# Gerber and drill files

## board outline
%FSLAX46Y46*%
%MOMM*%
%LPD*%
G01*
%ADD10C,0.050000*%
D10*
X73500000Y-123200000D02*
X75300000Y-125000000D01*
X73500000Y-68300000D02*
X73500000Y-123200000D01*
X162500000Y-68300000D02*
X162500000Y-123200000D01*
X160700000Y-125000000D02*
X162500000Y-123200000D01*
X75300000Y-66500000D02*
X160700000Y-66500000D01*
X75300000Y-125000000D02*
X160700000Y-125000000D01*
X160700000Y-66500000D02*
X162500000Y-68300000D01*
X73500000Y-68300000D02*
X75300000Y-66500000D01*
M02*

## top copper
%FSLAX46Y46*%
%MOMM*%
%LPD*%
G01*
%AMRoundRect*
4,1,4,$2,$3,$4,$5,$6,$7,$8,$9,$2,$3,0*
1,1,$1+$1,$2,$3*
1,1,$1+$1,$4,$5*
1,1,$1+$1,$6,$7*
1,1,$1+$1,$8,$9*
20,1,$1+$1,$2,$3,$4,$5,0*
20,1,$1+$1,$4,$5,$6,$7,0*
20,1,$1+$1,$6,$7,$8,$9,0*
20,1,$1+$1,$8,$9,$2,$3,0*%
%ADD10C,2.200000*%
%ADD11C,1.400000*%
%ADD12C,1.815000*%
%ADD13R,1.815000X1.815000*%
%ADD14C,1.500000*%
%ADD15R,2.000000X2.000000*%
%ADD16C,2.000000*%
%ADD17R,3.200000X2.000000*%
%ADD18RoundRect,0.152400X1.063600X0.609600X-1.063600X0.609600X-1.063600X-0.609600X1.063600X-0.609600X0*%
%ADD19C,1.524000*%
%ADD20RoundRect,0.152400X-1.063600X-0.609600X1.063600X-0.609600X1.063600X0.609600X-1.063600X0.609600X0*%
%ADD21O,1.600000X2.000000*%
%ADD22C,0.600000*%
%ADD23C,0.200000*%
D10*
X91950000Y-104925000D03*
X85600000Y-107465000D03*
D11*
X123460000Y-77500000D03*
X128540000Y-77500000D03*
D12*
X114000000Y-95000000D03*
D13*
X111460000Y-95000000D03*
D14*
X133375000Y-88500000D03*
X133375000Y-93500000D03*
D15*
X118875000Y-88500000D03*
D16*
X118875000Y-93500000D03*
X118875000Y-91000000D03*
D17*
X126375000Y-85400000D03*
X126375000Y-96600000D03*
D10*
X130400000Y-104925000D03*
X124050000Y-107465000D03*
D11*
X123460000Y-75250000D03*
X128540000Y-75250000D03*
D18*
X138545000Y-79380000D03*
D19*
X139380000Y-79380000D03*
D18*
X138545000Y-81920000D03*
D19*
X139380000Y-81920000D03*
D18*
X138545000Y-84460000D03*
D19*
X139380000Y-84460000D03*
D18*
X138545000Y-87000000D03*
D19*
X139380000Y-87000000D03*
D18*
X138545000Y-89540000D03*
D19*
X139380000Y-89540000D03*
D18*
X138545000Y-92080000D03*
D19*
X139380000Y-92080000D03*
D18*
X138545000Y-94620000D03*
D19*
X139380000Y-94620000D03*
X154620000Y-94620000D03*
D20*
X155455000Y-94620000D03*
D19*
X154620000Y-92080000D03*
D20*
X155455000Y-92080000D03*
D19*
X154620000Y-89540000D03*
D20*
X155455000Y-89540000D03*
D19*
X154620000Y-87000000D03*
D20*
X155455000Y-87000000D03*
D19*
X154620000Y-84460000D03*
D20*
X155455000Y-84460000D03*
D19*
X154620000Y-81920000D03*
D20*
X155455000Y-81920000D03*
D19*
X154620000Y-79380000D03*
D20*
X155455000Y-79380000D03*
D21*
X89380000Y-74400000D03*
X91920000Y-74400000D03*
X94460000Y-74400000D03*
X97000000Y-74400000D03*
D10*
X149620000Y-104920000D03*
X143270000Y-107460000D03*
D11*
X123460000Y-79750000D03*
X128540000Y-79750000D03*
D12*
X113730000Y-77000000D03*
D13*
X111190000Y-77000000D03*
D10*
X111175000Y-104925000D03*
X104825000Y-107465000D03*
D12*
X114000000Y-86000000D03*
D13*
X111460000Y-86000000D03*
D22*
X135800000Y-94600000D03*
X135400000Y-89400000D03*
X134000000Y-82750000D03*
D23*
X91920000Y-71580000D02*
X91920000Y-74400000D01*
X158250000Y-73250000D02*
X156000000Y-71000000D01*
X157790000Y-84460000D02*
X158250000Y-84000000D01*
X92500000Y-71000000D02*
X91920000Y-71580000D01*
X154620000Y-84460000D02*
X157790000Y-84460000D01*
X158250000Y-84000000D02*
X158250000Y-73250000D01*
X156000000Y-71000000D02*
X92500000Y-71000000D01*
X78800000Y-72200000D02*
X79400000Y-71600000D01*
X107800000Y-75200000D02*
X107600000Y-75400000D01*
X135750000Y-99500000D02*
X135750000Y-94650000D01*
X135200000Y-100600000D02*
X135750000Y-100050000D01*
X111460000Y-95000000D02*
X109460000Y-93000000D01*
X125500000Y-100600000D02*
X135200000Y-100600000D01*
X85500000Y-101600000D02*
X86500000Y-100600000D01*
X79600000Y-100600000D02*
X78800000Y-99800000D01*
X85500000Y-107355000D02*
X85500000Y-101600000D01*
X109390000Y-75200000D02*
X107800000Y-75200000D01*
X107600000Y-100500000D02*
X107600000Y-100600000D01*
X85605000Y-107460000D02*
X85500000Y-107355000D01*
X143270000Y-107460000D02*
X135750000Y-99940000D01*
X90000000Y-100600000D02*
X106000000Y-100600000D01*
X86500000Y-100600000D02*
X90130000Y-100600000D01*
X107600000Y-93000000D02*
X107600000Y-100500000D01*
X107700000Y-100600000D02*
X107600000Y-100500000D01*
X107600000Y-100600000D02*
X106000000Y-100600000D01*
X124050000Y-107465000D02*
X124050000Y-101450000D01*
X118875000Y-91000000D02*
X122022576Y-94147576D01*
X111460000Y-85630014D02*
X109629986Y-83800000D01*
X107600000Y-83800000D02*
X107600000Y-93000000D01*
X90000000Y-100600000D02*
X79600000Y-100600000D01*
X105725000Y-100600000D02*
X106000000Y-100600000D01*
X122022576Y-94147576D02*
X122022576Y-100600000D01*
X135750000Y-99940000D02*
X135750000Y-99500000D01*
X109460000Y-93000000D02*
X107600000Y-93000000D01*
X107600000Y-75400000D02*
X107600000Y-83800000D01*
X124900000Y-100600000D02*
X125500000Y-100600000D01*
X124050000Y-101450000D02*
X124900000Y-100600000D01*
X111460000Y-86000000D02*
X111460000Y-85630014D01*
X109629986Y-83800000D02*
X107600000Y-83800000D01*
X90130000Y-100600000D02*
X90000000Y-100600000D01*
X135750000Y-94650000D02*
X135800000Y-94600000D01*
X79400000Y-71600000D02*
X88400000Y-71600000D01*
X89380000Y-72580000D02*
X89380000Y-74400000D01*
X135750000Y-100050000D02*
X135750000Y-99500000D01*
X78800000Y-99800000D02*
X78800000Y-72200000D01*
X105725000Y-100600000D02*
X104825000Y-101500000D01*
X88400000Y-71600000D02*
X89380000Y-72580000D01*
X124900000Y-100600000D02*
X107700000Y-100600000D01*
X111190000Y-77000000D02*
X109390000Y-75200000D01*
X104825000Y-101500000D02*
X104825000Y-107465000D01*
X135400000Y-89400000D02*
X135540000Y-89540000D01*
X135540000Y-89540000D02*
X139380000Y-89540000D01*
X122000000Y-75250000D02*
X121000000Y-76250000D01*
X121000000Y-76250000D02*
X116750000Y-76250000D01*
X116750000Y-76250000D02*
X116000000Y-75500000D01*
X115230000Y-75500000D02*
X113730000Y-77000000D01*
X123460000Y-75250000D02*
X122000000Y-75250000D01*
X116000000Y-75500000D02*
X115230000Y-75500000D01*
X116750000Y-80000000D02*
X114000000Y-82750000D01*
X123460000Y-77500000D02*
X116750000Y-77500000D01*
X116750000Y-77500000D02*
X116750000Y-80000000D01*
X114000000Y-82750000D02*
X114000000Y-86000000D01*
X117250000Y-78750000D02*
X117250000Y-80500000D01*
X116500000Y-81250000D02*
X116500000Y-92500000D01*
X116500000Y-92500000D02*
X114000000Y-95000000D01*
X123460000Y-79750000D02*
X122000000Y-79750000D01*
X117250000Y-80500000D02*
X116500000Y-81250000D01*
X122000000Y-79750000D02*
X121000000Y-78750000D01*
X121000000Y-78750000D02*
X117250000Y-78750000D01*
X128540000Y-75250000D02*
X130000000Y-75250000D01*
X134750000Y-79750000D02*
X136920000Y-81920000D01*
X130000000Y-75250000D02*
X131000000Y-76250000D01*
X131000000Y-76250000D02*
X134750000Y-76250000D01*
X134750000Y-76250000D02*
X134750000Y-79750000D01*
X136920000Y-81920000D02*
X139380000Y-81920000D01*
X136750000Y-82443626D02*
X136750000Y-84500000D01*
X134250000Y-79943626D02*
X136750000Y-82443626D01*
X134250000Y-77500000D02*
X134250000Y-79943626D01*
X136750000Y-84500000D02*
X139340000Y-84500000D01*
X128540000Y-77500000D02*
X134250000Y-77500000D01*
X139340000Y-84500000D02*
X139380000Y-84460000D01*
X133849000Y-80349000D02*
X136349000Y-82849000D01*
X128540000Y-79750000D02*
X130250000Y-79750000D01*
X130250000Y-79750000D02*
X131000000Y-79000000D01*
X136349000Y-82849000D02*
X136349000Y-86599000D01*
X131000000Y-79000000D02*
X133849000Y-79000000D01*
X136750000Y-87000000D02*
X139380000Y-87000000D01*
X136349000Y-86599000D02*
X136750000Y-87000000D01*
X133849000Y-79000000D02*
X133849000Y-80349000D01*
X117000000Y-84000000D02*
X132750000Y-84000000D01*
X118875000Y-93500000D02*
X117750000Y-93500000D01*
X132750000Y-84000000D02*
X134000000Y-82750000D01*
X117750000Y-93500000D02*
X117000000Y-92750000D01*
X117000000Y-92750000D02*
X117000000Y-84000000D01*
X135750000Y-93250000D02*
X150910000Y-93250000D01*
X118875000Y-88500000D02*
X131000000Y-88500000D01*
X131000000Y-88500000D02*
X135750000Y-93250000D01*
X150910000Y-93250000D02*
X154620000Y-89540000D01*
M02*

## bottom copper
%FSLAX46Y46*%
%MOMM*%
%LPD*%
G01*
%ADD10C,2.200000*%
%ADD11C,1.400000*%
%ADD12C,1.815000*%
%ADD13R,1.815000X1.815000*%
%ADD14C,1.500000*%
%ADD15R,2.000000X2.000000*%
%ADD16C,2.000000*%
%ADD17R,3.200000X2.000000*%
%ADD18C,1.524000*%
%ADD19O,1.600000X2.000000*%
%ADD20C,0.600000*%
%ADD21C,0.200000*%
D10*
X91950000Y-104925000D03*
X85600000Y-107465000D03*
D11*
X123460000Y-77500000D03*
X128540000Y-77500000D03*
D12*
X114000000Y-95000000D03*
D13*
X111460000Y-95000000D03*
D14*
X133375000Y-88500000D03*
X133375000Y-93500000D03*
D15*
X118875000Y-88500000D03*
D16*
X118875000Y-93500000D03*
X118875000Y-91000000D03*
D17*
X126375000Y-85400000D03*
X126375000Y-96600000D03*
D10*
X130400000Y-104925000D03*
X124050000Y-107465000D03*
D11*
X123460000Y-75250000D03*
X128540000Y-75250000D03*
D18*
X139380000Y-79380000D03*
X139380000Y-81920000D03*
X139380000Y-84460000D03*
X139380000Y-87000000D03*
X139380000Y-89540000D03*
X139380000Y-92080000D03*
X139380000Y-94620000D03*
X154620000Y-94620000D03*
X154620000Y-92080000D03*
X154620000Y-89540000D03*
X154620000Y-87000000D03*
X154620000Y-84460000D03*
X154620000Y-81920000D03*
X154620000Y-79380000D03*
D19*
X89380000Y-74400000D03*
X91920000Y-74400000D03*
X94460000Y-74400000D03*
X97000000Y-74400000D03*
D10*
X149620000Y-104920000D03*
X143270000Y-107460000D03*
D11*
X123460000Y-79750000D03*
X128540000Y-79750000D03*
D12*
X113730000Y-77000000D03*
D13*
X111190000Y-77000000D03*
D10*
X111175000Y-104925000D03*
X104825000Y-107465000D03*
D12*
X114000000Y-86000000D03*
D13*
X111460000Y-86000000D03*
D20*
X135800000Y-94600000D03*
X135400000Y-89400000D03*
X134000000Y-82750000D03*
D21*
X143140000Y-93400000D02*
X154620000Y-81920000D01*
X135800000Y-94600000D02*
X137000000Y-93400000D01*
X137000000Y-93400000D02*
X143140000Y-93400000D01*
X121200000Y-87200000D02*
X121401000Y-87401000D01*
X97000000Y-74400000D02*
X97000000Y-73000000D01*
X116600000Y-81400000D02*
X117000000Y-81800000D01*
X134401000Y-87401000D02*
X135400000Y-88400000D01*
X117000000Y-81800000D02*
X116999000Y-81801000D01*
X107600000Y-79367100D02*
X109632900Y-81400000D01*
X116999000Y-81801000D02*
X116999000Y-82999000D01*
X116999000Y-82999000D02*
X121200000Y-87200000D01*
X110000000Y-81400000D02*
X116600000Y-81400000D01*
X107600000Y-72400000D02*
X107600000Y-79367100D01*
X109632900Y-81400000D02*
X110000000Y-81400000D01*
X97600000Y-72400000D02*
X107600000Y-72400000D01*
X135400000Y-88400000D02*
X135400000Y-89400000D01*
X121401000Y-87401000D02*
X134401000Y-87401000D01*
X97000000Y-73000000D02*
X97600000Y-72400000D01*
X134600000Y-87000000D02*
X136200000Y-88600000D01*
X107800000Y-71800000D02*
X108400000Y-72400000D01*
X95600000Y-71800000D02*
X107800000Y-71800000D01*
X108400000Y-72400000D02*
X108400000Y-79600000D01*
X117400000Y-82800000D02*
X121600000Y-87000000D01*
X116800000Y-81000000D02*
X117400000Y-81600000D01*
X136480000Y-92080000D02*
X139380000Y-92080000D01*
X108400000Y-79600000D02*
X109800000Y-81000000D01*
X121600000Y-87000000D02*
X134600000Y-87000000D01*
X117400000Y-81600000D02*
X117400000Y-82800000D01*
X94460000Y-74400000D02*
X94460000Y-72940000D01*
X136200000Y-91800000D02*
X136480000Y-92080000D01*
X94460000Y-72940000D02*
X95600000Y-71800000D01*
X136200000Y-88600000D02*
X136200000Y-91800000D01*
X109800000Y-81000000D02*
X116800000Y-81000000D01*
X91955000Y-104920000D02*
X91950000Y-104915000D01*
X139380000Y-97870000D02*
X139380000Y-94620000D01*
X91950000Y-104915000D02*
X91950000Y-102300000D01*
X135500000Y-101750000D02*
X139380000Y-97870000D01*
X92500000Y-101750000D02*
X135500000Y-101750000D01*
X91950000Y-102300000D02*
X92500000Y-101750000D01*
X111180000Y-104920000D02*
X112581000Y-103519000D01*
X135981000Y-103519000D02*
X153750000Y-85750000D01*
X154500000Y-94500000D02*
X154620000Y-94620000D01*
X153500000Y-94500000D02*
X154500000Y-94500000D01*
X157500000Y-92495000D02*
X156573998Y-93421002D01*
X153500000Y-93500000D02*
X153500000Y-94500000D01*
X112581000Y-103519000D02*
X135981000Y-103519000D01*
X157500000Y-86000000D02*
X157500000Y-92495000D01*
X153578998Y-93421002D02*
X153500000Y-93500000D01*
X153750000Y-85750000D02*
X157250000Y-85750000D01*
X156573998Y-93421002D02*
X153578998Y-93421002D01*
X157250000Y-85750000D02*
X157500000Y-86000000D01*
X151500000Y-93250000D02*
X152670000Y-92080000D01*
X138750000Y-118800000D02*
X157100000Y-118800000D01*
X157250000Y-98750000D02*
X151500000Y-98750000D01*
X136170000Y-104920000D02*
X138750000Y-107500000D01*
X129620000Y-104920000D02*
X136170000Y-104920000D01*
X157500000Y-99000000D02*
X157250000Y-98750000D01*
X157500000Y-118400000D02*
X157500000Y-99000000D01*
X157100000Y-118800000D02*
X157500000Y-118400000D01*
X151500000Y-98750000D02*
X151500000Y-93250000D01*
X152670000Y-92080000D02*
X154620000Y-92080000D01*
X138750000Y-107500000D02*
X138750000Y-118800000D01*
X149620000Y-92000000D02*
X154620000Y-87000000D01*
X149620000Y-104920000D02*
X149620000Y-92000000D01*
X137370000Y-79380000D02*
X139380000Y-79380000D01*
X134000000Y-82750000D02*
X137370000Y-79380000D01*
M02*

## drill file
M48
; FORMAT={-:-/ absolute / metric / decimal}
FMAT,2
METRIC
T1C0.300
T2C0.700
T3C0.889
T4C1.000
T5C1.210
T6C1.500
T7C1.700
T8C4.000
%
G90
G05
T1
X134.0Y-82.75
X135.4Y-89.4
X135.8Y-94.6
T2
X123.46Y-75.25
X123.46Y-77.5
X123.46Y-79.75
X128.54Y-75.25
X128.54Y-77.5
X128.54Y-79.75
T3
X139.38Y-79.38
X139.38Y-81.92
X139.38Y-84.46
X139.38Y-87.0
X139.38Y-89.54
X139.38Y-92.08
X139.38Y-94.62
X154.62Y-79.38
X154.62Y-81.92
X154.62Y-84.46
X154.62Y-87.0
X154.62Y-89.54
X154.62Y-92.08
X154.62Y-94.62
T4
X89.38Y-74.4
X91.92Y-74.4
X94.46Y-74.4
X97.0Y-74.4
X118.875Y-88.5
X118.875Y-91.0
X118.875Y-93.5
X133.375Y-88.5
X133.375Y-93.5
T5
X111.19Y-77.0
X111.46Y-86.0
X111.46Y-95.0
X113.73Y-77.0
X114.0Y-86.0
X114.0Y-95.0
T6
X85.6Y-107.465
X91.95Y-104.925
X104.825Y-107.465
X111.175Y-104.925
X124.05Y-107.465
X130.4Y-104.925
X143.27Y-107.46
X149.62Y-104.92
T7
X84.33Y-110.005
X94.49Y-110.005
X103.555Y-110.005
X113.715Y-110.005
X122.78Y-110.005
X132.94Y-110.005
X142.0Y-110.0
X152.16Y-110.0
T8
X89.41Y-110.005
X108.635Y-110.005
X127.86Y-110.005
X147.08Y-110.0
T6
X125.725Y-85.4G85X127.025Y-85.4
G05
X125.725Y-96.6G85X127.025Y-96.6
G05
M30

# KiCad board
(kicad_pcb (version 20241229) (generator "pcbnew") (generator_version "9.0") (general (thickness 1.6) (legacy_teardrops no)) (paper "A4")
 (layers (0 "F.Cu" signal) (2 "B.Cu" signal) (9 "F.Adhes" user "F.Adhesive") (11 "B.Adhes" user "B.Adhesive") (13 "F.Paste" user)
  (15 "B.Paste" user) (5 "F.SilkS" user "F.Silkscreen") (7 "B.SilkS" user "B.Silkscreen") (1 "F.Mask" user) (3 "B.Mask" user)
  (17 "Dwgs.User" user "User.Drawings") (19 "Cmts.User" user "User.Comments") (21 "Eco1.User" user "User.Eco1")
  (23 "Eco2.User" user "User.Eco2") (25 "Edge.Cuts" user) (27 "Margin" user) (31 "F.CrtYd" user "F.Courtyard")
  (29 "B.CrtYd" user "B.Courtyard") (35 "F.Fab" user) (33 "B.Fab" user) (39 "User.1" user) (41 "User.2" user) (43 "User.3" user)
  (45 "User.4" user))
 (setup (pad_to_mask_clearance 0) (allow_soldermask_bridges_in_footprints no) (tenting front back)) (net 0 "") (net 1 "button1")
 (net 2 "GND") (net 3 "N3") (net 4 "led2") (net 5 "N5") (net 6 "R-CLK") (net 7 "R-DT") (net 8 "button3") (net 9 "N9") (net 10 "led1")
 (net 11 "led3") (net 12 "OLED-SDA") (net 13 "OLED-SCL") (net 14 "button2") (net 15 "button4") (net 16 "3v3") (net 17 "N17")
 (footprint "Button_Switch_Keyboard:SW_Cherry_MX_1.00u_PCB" (layer "F.Cu") (at 91.95 104.925)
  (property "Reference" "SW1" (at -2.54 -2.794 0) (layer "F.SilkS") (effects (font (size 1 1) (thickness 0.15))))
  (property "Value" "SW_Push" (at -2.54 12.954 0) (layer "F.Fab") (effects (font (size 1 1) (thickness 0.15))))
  (pad "" np_thru_hole circle (at -7.62 5.08) (size 1.7 1.7) (drill 1.7) (layers "*.Cu" "*.Mask"))
  (pad "" np_thru_hole circle (at -2.54 5.08) (size 4 4) (drill 4) (layers "*.Cu" "*.Mask"))
  (pad "" np_thru_hole circle (at 2.54 5.08) (size 1.7 1.7) (drill 1.7) (layers "*.Cu" "*.Mask"))
  (pad "1" thru_hole circle (at 0 0) (size 2.2 2.2) (drill 1.5) (layers "*.Cu" "*.Mask") (remove_unused_layers no) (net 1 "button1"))
  (pad "2" thru_hole circle (at -6.35 2.54) (size 2.2 2.2) (drill 1.5) (layers "*.Cu" "*.Mask") (remove_unused_layers no) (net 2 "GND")))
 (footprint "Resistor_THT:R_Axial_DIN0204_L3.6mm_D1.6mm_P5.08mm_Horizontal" (layer "F.Cu") (at 123.46 77.5)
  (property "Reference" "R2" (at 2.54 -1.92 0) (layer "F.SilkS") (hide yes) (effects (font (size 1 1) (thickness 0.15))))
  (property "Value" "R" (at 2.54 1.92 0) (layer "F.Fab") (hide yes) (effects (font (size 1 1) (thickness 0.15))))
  (pad "1" thru_hole circle (at 0 0) (size 1.4 1.4) (drill 0.7) (layers "*.Cu" "*.Mask") (remove_unused_layers no) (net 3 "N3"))
  (pad "2" thru_hole circle (at 5.08 0) (size 1.4 1.4) (drill 0.7) (layers "*.Cu" "*.Mask") (remove_unused_layers no) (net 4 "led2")))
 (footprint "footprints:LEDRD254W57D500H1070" (layer "F.Cu") (at 112.73 95)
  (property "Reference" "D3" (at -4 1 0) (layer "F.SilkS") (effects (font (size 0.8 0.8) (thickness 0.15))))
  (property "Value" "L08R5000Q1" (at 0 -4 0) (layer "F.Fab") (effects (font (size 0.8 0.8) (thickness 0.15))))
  (pad "A" thru_hole circle (at 1.27 0) (size 1.815 1.815) (drill 1.21) (layers "*.Cu" "*.Mask") (remove_unused_layers no) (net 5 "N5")
   (solder_mask_margin 0.102))
  (pad "C" thru_hole rect (at -1.27 0) (size 1.815 1.815) (drill 1.21) (layers "*.Cu" "*.Mask") (remove_unused_layers no) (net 2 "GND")
   (solder_mask_margin 0.102)))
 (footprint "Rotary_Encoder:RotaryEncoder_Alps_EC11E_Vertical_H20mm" (layer "F.Cu") (at 118.875 88.5)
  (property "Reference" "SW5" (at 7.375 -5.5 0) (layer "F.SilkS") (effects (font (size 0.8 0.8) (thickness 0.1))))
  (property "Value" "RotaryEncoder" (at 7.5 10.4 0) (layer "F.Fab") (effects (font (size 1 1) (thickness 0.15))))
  (pad "" thru_hole circle (at 14.5 0) (size 1.5 1.5) (drill 1) (layers "*.Cu" "*.Mask") (remove_unused_layers no))
  (pad "" thru_hole circle (at 14.5 5) (size 1.5 1.5) (drill 1) (layers "*.Cu" "*.Mask") (remove_unused_layers no))
  (pad "A" thru_hole rect (at 0 0) (size 2 2) (drill 1) (layers "*.Cu" "*.Mask") (remove_unused_layers no) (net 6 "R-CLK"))
  (pad "B" thru_hole circle (at 0 5) (size 2 2) (drill 1) (layers "*.Cu" "*.Mask") (remove_unused_layers no) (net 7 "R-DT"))
  (pad "C" thru_hole circle (at 0 2.5) (size 2 2) (drill 1) (layers "*.Cu" "*.Mask") (remove_unused_layers no) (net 2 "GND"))
  (pad "MP" thru_hole rect (at 7.5 -3.1) (size 3.2 2) (drill oval 2.8 1.5) (layers "*.Cu" "*.Mask") (remove_unused_layers no))
  (pad "MP" thru_hole rect (at 7.5 8.1) (size 3.2 2) (drill oval 2.8 1.5) (layers "*.Cu" "*.Mask") (remove_unused_layers no)))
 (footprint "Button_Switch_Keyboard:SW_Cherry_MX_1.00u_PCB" (layer "F.Cu") (at 130.4 104.925)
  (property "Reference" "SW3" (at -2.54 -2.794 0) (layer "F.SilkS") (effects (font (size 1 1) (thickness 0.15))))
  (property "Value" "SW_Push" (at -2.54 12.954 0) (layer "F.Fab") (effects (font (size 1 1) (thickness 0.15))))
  (pad "" np_thru_hole circle (at -7.62 5.08) (size 1.7 1.7) (drill 1.7) (layers "*.Cu" "*.Mask"))
  (pad "" np_thru_hole circle (at -2.54 5.08) (size 4 4) (drill 4) (layers "*.Cu" "*.Mask"))
  (pad "" np_thru_hole circle (at 2.54 5.08) (size 1.7 1.7) (drill 1.7) (layers "*.Cu" "*.Mask"))
  (pad "1" thru_hole circle (at 0 0) (size 2.2 2.2) (drill 1.5) (layers "*.Cu" "*.Mask") (remove_unused_layers no) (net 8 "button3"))
  (pad "2" thru_hole circle (at -6.35 2.54) (size 2.2 2.2) (drill 1.5) (layers "*.Cu" "*.Mask") (remove_unused_layers no) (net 2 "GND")))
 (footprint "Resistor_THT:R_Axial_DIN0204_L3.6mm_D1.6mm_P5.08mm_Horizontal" (layer "F.Cu") (at 123.46 75.25)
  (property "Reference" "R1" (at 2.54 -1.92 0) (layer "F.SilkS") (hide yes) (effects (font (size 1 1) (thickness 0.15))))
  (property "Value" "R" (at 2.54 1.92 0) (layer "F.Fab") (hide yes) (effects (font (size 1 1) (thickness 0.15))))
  (pad "1" thru_hole circle (at 0 0) (size 1.4 1.4) (drill 0.7) (layers "*.Cu" "*.Mask") (remove_unused_layers no) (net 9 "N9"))
  (pad "2" thru_hole circle (at 5.08 0) (size 1.4 1.4) (drill 0.7) (layers "*.Cu" "*.Mask") (remove_unused_layers no) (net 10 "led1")))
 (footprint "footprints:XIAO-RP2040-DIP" (layer "F.Cu") (at 147 87)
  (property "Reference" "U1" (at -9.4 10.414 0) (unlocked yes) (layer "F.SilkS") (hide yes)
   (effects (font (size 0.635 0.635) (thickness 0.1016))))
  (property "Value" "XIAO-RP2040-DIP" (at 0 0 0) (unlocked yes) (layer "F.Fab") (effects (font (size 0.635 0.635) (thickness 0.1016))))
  (pad "1" smd roundrect (at -8.455 -7.62 180) (size 2.432 1.524) (layers "F.Cu" "F.Mask") (roundrect_rratio 0.1) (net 7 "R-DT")
   (thermal_bridge_angle 45))
  (pad "1" thru_hole circle (at -7.62 -7.62 180) (size 1.524 1.524) (drill 0.889) (layers "*.Cu" "*.Mask") (remove_unused_layers no)
   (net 7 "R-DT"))
  (pad "2" smd roundrect (at -8.455 -5.08 180) (size 2.432 1.524) (layers "F.Cu" "F.Mask") (roundrect_rratio 0.1) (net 10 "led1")
   (thermal_bridge_angle 45))
  (pad "2" thru_hole circle (at -7.62 -5.08 180) (size 1.524 1.524) (drill 0.889) (layers "*.Cu" "*.Mask") (remove_unused_layers no)
   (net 10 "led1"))
  (pad "3" smd roundrect (at -8.455 -2.54 180) (size 2.432 1.524) (layers "F.Cu" "F.Mask") (roundrect_rratio 0.1) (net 4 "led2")
   (thermal_bridge_angle 45))
  (pad "3" thru_hole circle (at -7.62 -2.54 180) (size 1.524 1.524) (drill 0.889) (layers "*.Cu" "*.Mask") (remove_unused_layers no)
   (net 4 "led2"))
  (pad "4" smd roundrect (at -8.455 0 180) (size 2.432 1.524) (layers "F.Cu" "F.Mask") (roundrect_rratio 0.1) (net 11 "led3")
   (thermal_bridge_angle 45))
  (pad "4" thru_hole circle (at -7.62 0 180) (size 1.524 1.524) (drill 0.889) (layers "*.Cu" "*.Mask") (remove_unused_layers no)
   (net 11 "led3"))
  (pad "5" smd roundrect (at -8.455 2.54 180) (size 2.432 1.524) (layers "F.Cu" "F.Mask") (roundrect_rratio 0.1) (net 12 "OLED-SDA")
   (thermal_bridge_angle 45))
  (pad "5" thru_hole circle (at -7.62 2.54 180) (size 1.524 1.524) (drill 0.889) (layers "*.Cu" "*.Mask") (remove_unused_layers no)
   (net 12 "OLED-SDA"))
  (pad "6" smd roundrect (at -8.455 5.08 180) (size 2.432 1.524) (layers "F.Cu" "F.Mask") (roundrect_rratio 0.1) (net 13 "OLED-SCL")
   (thermal_bridge_angle 45))
  (pad "6" thru_hole circle (at -7.62 5.08 180) (size 1.524 1.524) (drill 0.889) (layers "*.Cu" "*.Mask") (remove_unused_layers no)
   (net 13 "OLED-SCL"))
  (pad "7" smd roundrect (at -8.455 7.62 180) (size 2.432 1.524) (layers "F.Cu" "F.Mask") (roundrect_rratio 0.1) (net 1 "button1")
   (thermal_bridge_angle 45))
  (pad "7" thru_hole circle (at -7.62 7.62 180) (size 1.524 1.524) (drill 0.889) (layers "*.Cu" "*.Mask") (remove_unused_layers no)
   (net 1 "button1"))
  (pad "8" thru_hole circle (at 7.62 7.62) (size 1.524 1.524) (drill 0.889) (layers "*.Cu" "*.Mask") (remove_unused_layers no)
   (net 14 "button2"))
  (pad "8" smd roundrect (at 8.455 7.62) (size 2.432 1.524) (layers "F.Cu" "F.Mask") (roundrect_rratio 0.1) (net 14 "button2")
   (thermal_bridge_angle 45))
  (pad "9" thru_hole circle (at 7.62 5.08) (size 1.524 1.524) (drill 0.889) (layers "*.Cu" "*.Mask") (remove_unused_layers no)
   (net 8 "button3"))
  (pad "9" smd roundrect (at 8.455 5.08) (size 2.432 1.524) (layers "F.Cu" "F.Mask") (roundrect_rratio 0.1) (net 8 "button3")
   (thermal_bridge_angle 45))
  (pad "10" thru_hole circle (at 7.62 2.54) (size 1.524 1.524) (drill 0.889) (layers "*.Cu" "*.Mask") (remove_unused_layers no)
   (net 6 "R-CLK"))
  (pad "10" smd roundrect (at 8.455 2.54) (size 2.432 1.524) (layers "F.Cu" "F.Mask") (roundrect_rratio 0.1) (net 6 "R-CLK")
   (thermal_bridge_angle 45))
  (pad "11" thru_hole circle (at 7.62 0) (size 1.524 1.524) (drill 0.889) (layers "*.Cu" "*.Mask") (remove_unused_layers no)
   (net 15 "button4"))
  (pad "11" smd roundrect (at 8.455 0) (size 2.432 1.524) (layers "F.Cu" "F.Mask") (roundrect_rratio 0.1) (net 15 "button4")
   (thermal_bridge_angle 45))
  (pad "12" thru_hole circle (at 7.62 -2.54) (size 1.524 1.524) (drill 0.889) (layers "*.Cu" "*.Mask") (remove_unused_layers no)
   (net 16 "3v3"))
  (pad "12" smd roundrect (at 8.455 -2.54) (size 2.432 1.524) (layers "F.Cu" "F.Mask") (roundrect_rratio 0.1) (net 16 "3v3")
   (thermal_bridge_angle 45))
  (pad "13" thru_hole circle (at 7.62 -5.08) (size 1.524 1.524) (drill 0.889) (layers "*.Cu" "*.Mask") (remove_unused_layers no)
   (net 2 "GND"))
  (pad "13" smd roundrect (at 8.455 -5.08) (size 2.432 1.524) (layers "F.Cu" "F.Mask") (roundrect_rratio 0.1) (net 2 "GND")
   (thermal_bridge_angle 45))
  (pad "14" thru_hole circle (at 7.62 -7.62) (size 1.524 1.524) (drill 0.889) (layers "*.Cu" "*.Mask") (remove_unused_layers no)
   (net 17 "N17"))
  (pad "14" smd roundrect (at 8.455 -7.62) (size 2.432 1.524) (layers "F.Cu" "F.Mask") (roundrect_rratio 0.1) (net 17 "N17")
   (thermal_bridge_angle 45)))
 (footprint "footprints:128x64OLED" (layer "F.Cu") (at 93 85)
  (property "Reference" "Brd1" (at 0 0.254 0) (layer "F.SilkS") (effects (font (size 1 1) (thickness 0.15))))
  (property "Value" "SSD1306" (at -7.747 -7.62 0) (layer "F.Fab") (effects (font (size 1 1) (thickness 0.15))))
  (pad "1" thru_hole oval (at -3.62 -10.6 90) (size 2 1.6) (drill 1) (layers "*.Cu" "*.Mask") (remove_unused_layers no) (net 2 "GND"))
  (pad "2" thru_hole oval (at -1.08 -10.6 90) (size 2 1.6) (drill 1) (layers "*.Cu" "*.Mask") (remove_unused_layers no) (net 16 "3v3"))
  (pad "3" thru_hole oval (at 1.46 -10.6 90) (size 2 1.6) (drill 1) (layers "*.Cu" "*.Mask") (remove_unused_layers no) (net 13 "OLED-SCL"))
  (pad "4" thru_hole oval (at 4 -10.6 90) (size 2 1.6) (drill 1) (layers "*.Cu" "*.Mask") (remove_unused_layers no) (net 12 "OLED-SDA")))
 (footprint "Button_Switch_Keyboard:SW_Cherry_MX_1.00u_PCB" (layer "F.Cu") (at 149.62 104.92)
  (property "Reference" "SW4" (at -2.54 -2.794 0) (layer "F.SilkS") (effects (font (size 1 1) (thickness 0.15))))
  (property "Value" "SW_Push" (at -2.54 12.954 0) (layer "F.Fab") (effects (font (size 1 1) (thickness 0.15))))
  (pad "" np_thru_hole circle (at -7.62 5.08) (size 1.7 1.7) (drill 1.7) (layers "*.Cu" "*.Mask"))
  (pad "" np_thru_hole circle (at -2.54 5.08) (size 4 4) (drill 4) (layers "*.Cu" "*.Mask"))
  (pad "" np_thru_hole circle (at 2.54 5.08) (size 1.7 1.7) (drill 1.7) (layers "*.Cu" "*.Mask"))
  (pad "1" thru_hole circle (at 0 0) (size 2.2 2.2) (drill 1.5) (layers "*.Cu" "*.Mask") (remove_unused_layers no) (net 15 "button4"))
  (pad "2" thru_hole circle (at -6.35 2.54) (size 2.2 2.2) (drill 1.5) (layers "*.Cu" "*.Mask") (remove_unused_layers no) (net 2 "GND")))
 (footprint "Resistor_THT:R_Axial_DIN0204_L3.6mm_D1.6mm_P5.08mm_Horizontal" (layer "F.Cu") (at 123.46 79.75)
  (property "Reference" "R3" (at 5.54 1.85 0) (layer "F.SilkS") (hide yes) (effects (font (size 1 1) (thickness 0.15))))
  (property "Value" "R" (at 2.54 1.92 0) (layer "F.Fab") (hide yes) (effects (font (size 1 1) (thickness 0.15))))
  (pad "1" thru_hole circle (at 0 0) (size 1.4 1.4) (drill 0.7) (layers "*.Cu" "*.Mask") (remove_unused_layers no) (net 5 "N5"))
  (pad "2" thru_hole circle (at 5.08 0) (size 1.4 1.4) (drill 0.7) (layers "*.Cu" "*.Mask") (remove_unused_layers no) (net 11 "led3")))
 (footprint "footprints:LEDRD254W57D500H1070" (layer "F.Cu") (at 112.46 77)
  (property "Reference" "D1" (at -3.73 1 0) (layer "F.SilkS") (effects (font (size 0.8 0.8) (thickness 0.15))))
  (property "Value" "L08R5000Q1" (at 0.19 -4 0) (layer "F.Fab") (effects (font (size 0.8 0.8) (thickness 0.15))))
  (pad "A" thru_hole circle (at 1.27 0) (size 1.815 1.815) (drill 1.21) (layers "*.Cu" "*.Mask") (remove_unused_layers no) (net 9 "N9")
   (solder_mask_margin 0.102))
  (pad "C" thru_hole rect (at -1.27 0) (size 1.815 1.815) (drill 1.21) (layers "*.Cu" "*.Mask") (remove_unused_layers no) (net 2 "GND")
   (solder_mask_margin 0.102)))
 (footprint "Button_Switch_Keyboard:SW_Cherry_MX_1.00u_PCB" (layer "F.Cu") (at 111.175 104.925)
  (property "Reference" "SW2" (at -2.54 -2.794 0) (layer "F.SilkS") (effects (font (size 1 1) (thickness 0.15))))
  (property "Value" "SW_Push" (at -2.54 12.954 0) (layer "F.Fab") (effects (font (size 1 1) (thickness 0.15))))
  (pad "" np_thru_hole circle (at -7.62 5.08) (size 1.7 1.7) (drill 1.7) (layers "*.Cu" "*.Mask"))
  (pad "" np_thru_hole circle (at -2.54 5.08) (size 4 4) (drill 4) (layers "*.Cu" "*.Mask"))
  (pad "" np_thru_hole circle (at 2.54 5.08) (size 1.7 1.7) (drill 1.7) (layers "*.Cu" "*.Mask"))
  (pad "1" thru_hole circle (at 0 0) (size 2.2 2.2) (drill 1.5) (layers "*.Cu" "*.Mask") (remove_unused_layers no) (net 14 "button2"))
  (pad "2" thru_hole circle (at -6.35 2.54) (size 2.2 2.2) (drill 1.5) (layers "*.Cu" "*.Mask") (remove_unused_layers no) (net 2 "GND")))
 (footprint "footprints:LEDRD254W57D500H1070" (layer "F.Cu") (at 112.73 86)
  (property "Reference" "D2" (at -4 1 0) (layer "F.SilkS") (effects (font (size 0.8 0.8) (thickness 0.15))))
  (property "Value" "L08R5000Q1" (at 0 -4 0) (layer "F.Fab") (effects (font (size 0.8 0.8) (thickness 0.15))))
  (pad "A" thru_hole circle (at 1.27 0) (size 1.815 1.815) (drill 1.21) (layers "*.Cu" "*.Mask") (remove_unused_layers no) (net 3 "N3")
   (solder_mask_margin 0.102))
  (pad "C" thru_hole rect (at -1.27 0) (size 1.815 1.815) (drill 1.21) (layers "*.Cu" "*.Mask") (remove_unused_layers no) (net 2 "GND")
   (solder_mask_margin 0.102)))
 (gr_line (start 73.5 123.2) (end 75.3 125) (stroke (width 0.05) (type default)) (layer "Edge.Cuts"))
 (gr_line (start 73.5 68.3) (end 73.5 123.2) (stroke (width 0.05) (type default)) (layer "Edge.Cuts"))
 (gr_line (start 162.5 68.3) (end 162.5 123.2) (stroke (width 0.05) (type default)) (layer "Edge.Cuts"))
 (gr_line (start 160.7 125) (end 162.5 123.2) (stroke (width 0.05) (type default)) (layer "Edge.Cuts"))
 (gr_line (start 75.3 66.5) (end 160.7 66.5) (stroke (width 0.05) (type default)) (layer "Edge.Cuts"))
 (gr_line (start 75.3 125) (end 160.7 125) (stroke (width 0.05) (type default)) (layer "Edge.Cuts"))
 (gr_line (start 160.7 66.5) (end 162.5 68.3) (stroke (width 0.05) (type default)) (layer "Edge.Cuts"))
 (gr_line (start 73.5 68.3) (end 75.3 66.5) (stroke (width 0.05) (type default)) (layer "Edge.Cuts"))
 (segment (start 91.92 71.58) (end 91.92 74.4) (width 0.2) (layer "F.Cu") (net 16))
 (segment (start 158.25 73.25) (end 156 71) (width 0.2) (layer "F.Cu") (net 16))
 (segment (start 157.79 84.46) (end 158.25 84) (width 0.2) (layer "F.Cu") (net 16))
 (segment (start 92.5 71) (end 91.92 71.58) (width 0.2) (layer "F.Cu") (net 16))
 (segment (start 154.62 84.46) (end 157.79 84.46) (width 0.2) (layer "F.Cu") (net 16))
 (segment (start 158.25 84) (end 158.25 73.25) (width 0.2) (layer "F.Cu") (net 16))
 (segment (start 156 71) (end 92.5 71) (width 0.2) (layer "F.Cu") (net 16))
 (segment (start 78.8 72.2) (end 79.4 71.6) (width 0.2) (layer "F.Cu") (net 2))
 (segment (start 107.8 75.2) (end 107.6 75.4) (width 0.2) (layer "F.Cu") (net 2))
 (segment (start 135.75 99.5) (end 135.75 94.65) (width 0.2) (layer "F.Cu") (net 2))
 (segment (start 135.2 100.6) (end 135.75 100.05) (width 0.2) (layer "F.Cu") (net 2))
 (segment (start 111.46 95) (end 109.46 93) (width 0.2) (layer "F.Cu") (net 2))
 (segment (start 125.5 100.6) (end 135.2 100.6) (width 0.2) (layer "F.Cu") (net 2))
 (segment (start 85.5 101.6) (end 86.5 100.6) (width 0.2) (layer "F.Cu") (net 2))
 (segment (start 79.6 100.6) (end 78.8 99.8) (width 0.2) (layer "F.Cu") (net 2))
 (segment (start 85.5 107.355) (end 85.5 101.6) (width 0.2) (layer "F.Cu") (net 2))
 (segment (start 109.39 75.2) (end 107.8 75.2) (width 0.2) (layer "F.Cu") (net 2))
 (segment (start 107.6 100.5) (end 107.6 100.6) (width 0.2) (layer "F.Cu") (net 2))
 (segment (start 85.605 107.46) (end 85.5 107.355) (width 0.2) (layer "F.Cu") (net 2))
 (segment (start 143.27 107.46) (end 135.75 99.94) (width 0.2) (layer "F.Cu") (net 2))
 (segment (start 90 100.6) (end 106 100.6) (width 0.2) (layer "F.Cu") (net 2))
 (segment (start 86.5 100.6) (end 90.13 100.6) (width 0.2) (layer "F.Cu") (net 2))
 (segment (start 107.6 93) (end 107.6 100.5) (width 0.2) (layer "F.Cu") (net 2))
 (segment (start 107.7 100.6) (end 107.6 100.5) (width 0.2) (layer "F.Cu") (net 2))
 (segment (start 107.6 100.6) (end 106 100.6) (width 0.2) (layer "F.Cu") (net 2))
 (segment (start 124.05 107.465) (end 124.05 101.45) (width 0.2) (layer "F.Cu") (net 2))
 (segment (start 118.875 91) (end 122.022576 94.147576) (width 0.2) (layer "F.Cu") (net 2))
 (segment (start 111.46 85.630014) (end 109.629986 83.8) (width 0.2) (layer "F.Cu") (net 2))
 (segment (start 107.6 83.8) (end 107.6 93) (width 0.2) (layer "F.Cu") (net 2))
 (segment (start 90 100.6) (end 79.6 100.6) (width 0.2) (layer "F.Cu") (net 2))
 (segment (start 105.725 100.6) (end 106 100.6) (width 0.2) (layer "F.Cu") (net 2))
 (segment (start 122.022576 94.147576) (end 122.022576 100.6) (width 0.2) (layer "F.Cu") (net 2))
 (segment (start 135.75 99.94) (end 135.75 99.5) (width 0.2) (layer "F.Cu") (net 2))
 (segment (start 109.46 93) (end 107.6 93) (width 0.2) (layer "F.Cu") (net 2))
 (segment (start 107.6 75.4) (end 107.6 83.8) (width 0.2) (layer "F.Cu") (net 2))
 (segment (start 124.9 100.6) (end 125.5 100.6) (width 0.2) (layer "F.Cu") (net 2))
 (segment (start 124.05 101.45) (end 124.9 100.6) (width 0.2) (layer "F.Cu") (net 2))
 (segment (start 111.46 86) (end 111.46 85.630014) (width 0.2) (layer "F.Cu") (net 2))
 (segment (start 109.629986 83.8) (end 107.6 83.8) (width 0.2) (layer "F.Cu") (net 2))
 (segment (start 90.13 100.6) (end 90 100.6) (width 0.2) (layer "F.Cu") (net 2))
 (segment (start 135.75 94.65) (end 135.8 94.6) (width 0.2) (layer "F.Cu") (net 2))
 (segment (start 79.4 71.6) (end 88.4 71.6) (width 0.2) (layer "F.Cu") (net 2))
 (segment (start 89.38 72.58) (end 89.38 74.4) (width 0.2) (layer "F.Cu") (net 2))
 (segment (start 135.75 100.05) (end 135.75 99.5) (width 0.2) (layer "F.Cu") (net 2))
 (segment (start 78.8 99.8) (end 78.8 72.2) (width 0.2) (layer "F.Cu") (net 2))
 (segment (start 105.725 100.6) (end 104.825 101.5) (width 0.2) (layer "F.Cu") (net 2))
 (segment (start 88.4 71.6) (end 89.38 72.58) (width 0.2) (layer "F.Cu") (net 2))
 (segment (start 124.9 100.6) (end 107.7 100.6) (width 0.2) (layer "F.Cu") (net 2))
 (segment (start 111.19 77) (end 109.39 75.2) (width 0.2) (layer "F.Cu") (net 2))
 (segment (start 104.825 101.5) (end 104.825 107.465) (width 0.2) (layer "F.Cu") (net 2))
 (via (at 135.8 94.6) (size 0.6) (drill 0.3) (layers "F.Cu" "B.Cu") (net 2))
 (segment (start 143.14 93.4) (end 154.62 81.92) (width 0.2) (layer "B.Cu") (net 2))
 (segment (start 135.8 94.6) (end 137 93.4) (width 0.2) (layer "B.Cu") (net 2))
 (segment (start 137 93.4) (end 143.14 93.4) (width 0.2) (layer "B.Cu") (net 2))
 (segment (start 135.4 89.4) (end 135.54 89.54) (width 0.2) (layer "F.Cu") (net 12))
 (segment (start 135.54 89.54) (end 139.38 89.54) (width 0.2) (layer "F.Cu") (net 12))
 (via (at 135.4 89.4) (size 0.6) (drill 0.3) (layers "F.Cu" "B.Cu") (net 12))
 (segment (start 121.2 87.2) (end 121.401 87.401) (width 0.2) (layer "B.Cu") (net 12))
 (segment (start 97 74.4) (end 97 73) (width 0.2) (layer "B.Cu") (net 12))
 (segment (start 116.6 81.4) (end 117 81.8) (width 0.2) (layer "B.Cu") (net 12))
 (segment (start 134.401 87.401) (end 135.4 88.4) (width 0.2) (layer "B.Cu") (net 12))
 (segment (start 117 81.8) (end 116.999 81.801) (width 0.2) (layer "B.Cu") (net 12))
 (segment (start 107.6 79.3671) (end 109.6329 81.4) (width 0.2) (layer "B.Cu") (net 12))
 (segment (start 116.999 81.801) (end 116.999 82.999) (width 0.2) (layer "B.Cu") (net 12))
 (segment (start 116.999 82.999) (end 121.2 87.2) (width 0.2) (layer "B.Cu") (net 12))
 (segment (start 110 81.4) (end 116.6 81.4) (width 0.2) (layer "B.Cu") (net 12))
 (segment (start 107.6 72.4) (end 107.6 79.3671) (width 0.2) (layer "B.Cu") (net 12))
 (segment (start 109.6329 81.4) (end 110 81.4) (width 0.2) (layer "B.Cu") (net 12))
 (segment (start 97.6 72.4) (end 107.6 72.4) (width 0.2) (layer "B.Cu") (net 12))
 (segment (start 135.4 88.4) (end 135.4 89.4) (width 0.2) (layer "B.Cu") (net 12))
 (segment (start 121.401 87.401) (end 134.401 87.401) (width 0.2) (layer "B.Cu") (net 12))
 (segment (start 97 73) (end 97.6 72.4) (width 0.2) (layer "B.Cu") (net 12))
 (segment (start 134.6 87) (end 136.2 88.6) (width 0.2) (layer "B.Cu") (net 13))
 (segment (start 107.8 71.8) (end 108.4 72.4) (width 0.2) (layer "B.Cu") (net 13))
 (segment (start 95.6 71.8) (end 107.8 71.8) (width 0.2) (layer "B.Cu") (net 13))
 (segment (start 108.4 72.4) (end 108.4 79.6) (width 0.2) (layer "B.Cu") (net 13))
 (segment (start 117.4 82.8) (end 121.6 87) (width 0.2) (layer "B.Cu") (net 13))
 (segment (start 116.8 81) (end 117.4 81.6) (width 0.2) (layer "B.Cu") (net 13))
 (segment (start 136.48 92.08) (end 139.38 92.08) (width 0.2) (layer "B.Cu") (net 13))
 (segment (start 108.4 79.6) (end 109.8 81) (width 0.2) (layer "B.Cu") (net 13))
 (segment (start 121.6 87) (end 134.6 87) (width 0.2) (layer "B.Cu") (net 13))
 (segment (start 117.4 81.6) (end 117.4 82.8) (width 0.2) (layer "B.Cu") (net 13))
 (segment (start 94.46 74.4) (end 94.46 72.94) (width 0.2) (layer "B.Cu") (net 13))
 (segment (start 136.2 91.8) (end 136.48 92.08) (width 0.2) (layer "B.Cu") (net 13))
 (segment (start 94.46 72.94) (end 95.6 71.8) (width 0.2) (layer "B.Cu") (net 13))
 (segment (start 136.2 88.6) (end 136.2 91.8) (width 0.2) (layer "B.Cu") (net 13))
 (segment (start 109.8 81) (end 116.8 81) (width 0.2) (layer "B.Cu") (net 13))
 (segment (start 122 75.25) (end 121 76.25) (width 0.2) (layer "F.Cu") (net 9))
 (segment (start 121 76.25) (end 116.75 76.25) (width 0.2) (layer "F.Cu") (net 9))
 (segment (start 116.75 76.25) (end 116 75.5) (width 0.2) (layer "F.Cu") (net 9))
 (segment (start 115.23 75.5) (end 113.73 77) (width 0.2) (layer "F.Cu") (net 9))
 (segment (start 123.46 75.25) (end 122 75.25) (width 0.2) (layer "F.Cu") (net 9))
 (segment (start 116 75.5) (end 115.23 75.5) (width 0.2) (layer "F.Cu") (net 9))
 (segment (start 116.75 80) (end 114 82.75) (width 0.2) (layer "F.Cu") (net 3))
 (segment (start 123.46 77.5) (end 116.75 77.5) (width 0.2) (layer "F.Cu") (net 3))
 (segment (start 116.75 77.5) (end 116.75 80) (width 0.2) (layer "F.Cu") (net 3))
 (segment (start 114 82.75) (end 114 86) (width 0.2) (layer "F.Cu") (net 3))
 (segment (start 117.25 78.75) (end 117.25 80.5) (width 0.2) (layer "F.Cu") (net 5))
 (segment (start 116.5 81.25) (end 116.5 92.5) (width 0.2) (layer "F.Cu") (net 5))
 (segment (start 116.5 92.5) (end 114 95) (width 0.2) (layer "F.Cu") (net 5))
 (segment (start 123.46 79.75) (end 122 79.75) (width 0.2) (layer "F.Cu") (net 5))
 (segment (start 117.25 80.5) (end 116.5 81.25) (width 0.2) (layer "F.Cu") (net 5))
 (segment (start 122 79.75) (end 121 78.75) (width 0.2) (layer "F.Cu") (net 5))
 (segment (start 121 78.75) (end 117.25 78.75) (width 0.2) (layer "F.Cu") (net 5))
 (segment (start 128.54 75.25) (end 130 75.25) (width 0.2) (layer "F.Cu") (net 10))
 (segment (start 134.75 79.75) (end 136.92 81.92) (width 0.2) (layer "F.Cu") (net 10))
 (segment (start 130 75.25) (end 131 76.25) (width 0.2) (layer "F.Cu") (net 10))
 (segment (start 131 76.25) (end 134.75 76.25) (width 0.2) (layer "F.Cu") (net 10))
 (segment (start 134.75 76.25) (end 134.75 79.75) (width 0.2) (layer "F.Cu") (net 10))
 (segment (start 136.92 81.92) (end 139.38 81.92) (width 0.2) (layer "F.Cu") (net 10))
 (segment (start 136.75 82.443626) (end 136.75 84.5) (width 0.2) (layer "F.Cu") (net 4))
 (segment (start 134.25 79.943626) (end 136.75 82.443626) (width 0.2) (layer "F.Cu") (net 4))
 (segment (start 134.25 77.5) (end 134.25 79.943626) (width 0.2) (layer "F.Cu") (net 4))
 (segment (start 136.75 84.5) (end 139.34 84.5) (width 0.2) (layer "F.Cu") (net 4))
 (segment (start 128.54 77.5) (end 134.25 77.5) (width 0.2) (layer "F.Cu") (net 4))
 (segment (start 139.34 84.5) (end 139.38 84.46) (width 0.2) (layer "F.Cu") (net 4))
 (segment (start 133.849 80.349) (end 136.349 82.849) (width 0.2) (layer "F.Cu") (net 11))
 (segment (start 128.54 79.75) (end 130.25 79.75) (width 0.2) (layer "F.Cu") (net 11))
 (segment (start 130.25 79.75) (end 131 79) (width 0.2) (layer "F.Cu") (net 11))
 (segment (start 136.349 82.849) (end 136.349 86.599) (width 0.2) (layer "F.Cu") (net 11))
 (segment (start 131 79) (end 133.849 79) (width 0.2) (layer "F.Cu") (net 11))
 (segment (start 136.75 87) (end 139.38 87) (width 0.2) (layer "F.Cu") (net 11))
 (segment (start 136.349 86.599) (end 136.75 87) (width 0.2) (layer "F.Cu") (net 11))
 (segment (start 133.849 79) (end 133.849 80.349) (width 0.2) (layer "F.Cu") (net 11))
 (segment (start 91.955 104.92) (end 91.95 104.915) (width 0.2) (layer "B.Cu") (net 1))
 (segment (start 139.38 97.87) (end 139.38 94.62) (width 0.2) (layer "B.Cu") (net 1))
 (segment (start 91.95 104.915) (end 91.95 102.3) (width 0.2) (layer "B.Cu") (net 1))
 (segment (start 135.5 101.75) (end 139.38 97.87) (width 0.2) (layer "B.Cu") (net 1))
 (segment (start 92.5 101.75) (end 135.5 101.75) (width 0.2) (layer "B.Cu") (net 1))
 (segment (start 91.95 102.3) (end 92.5 101.75) (width 0.2) (layer "B.Cu") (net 1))
 (segment (start 111.18 104.92) (end 112.581 103.519) (width 0.2) (layer "B.Cu") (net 14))
 (segment (start 135.981 103.519) (end 153.75 85.75) (width 0.2) (layer "B.Cu") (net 14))
 (segment (start 154.5 94.5) (end 154.62 94.62) (width 0.2) (layer "B.Cu") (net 14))
 (segment (start 153.5 94.5) (end 154.5 94.5) (width 0.2) (layer "B.Cu") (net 14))
 (segment (start 157.5 92.495) (end 156.573998 93.421002) (width 0.2) (layer "B.Cu") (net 14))
 (segment (start 153.5 93.5) (end 153.5 94.5) (width 0.2) (layer "B.Cu") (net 14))
 (segment (start 112.581 103.519) (end 135.981 103.519) (width 0.2) (layer "B.Cu") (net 14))
 (segment (start 157.5 86) (end 157.5 92.495) (width 0.2) (layer "B.Cu") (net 14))
 (segment (start 153.578998 93.421002) (end 153.5 93.5) (width 0.2) (layer "B.Cu") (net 14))
 (segment (start 153.75 85.75) (end 157.25 85.75) (width 0.2) (layer "B.Cu") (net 14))
 (segment (start 156.573998 93.421002) (end 153.578998 93.421002) (width 0.2) (layer "B.Cu") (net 14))
 (segment (start 157.25 85.75) (end 157.5 86) (width 0.2) (layer "B.Cu") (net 14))
 (segment (start 151.5 93.25) (end 152.67 92.08) (width 0.2) (layer "B.Cu") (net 8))
 (segment (start 138.75 118.8) (end 157.1 118.8) (width 0.2) (layer "B.Cu") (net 8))
 (segment (start 157.25 98.75) (end 151.5 98.75) (width 0.2) (layer "B.Cu") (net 8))
 (segment (start 136.17 104.92) (end 138.75 107.5) (width 0.2) (layer "B.Cu") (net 8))
 (segment (start 129.62 104.92) (end 136.17 104.92) (width 0.2) (layer "B.Cu") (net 8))
 (segment (start 157.5 99) (end 157.25 98.75) (width 0.2) (layer "B.Cu") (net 8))
 (segment (start 157.5 118.4) (end 157.5 99) (width 0.2) (layer "B.Cu") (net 8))
 (segment (start 157.1 118.8) (end 157.5 118.4) (width 0.2) (layer "B.Cu") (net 8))
 (segment (start 151.5 98.75) (end 151.5 93.25) (width 0.2) (layer "B.Cu") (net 8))
 (segment (start 152.67 92.08) (end 154.62 92.08) (width 0.2) (layer "B.Cu") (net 8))
 (segment (start 138.75 107.5) (end 138.75 118.8) (width 0.2) (layer "B.Cu") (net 8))
 (segment (start 149.62 92) (end 154.62 87) (width 0.2) (layer "B.Cu") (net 15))
 (segment (start 149.62 104.92) (end 149.62 92) (width 0.2) (layer "B.Cu") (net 15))
 (segment (start 117 84) (end 132.75 84) (width 0.2) (layer "F.Cu") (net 7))
 (segment (start 118.875 93.5) (end 117.75 93.5) (width 0.2) (layer "F.Cu") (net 7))
 (segment (start 132.75 84) (end 134 82.75) (width 0.2) (layer "F.Cu") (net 7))
 (segment (start 117.75 93.5) (end 117 92.75) (width 0.2) (layer "F.Cu") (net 7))
 (segment (start 117 92.75) (end 117 84) (width 0.2) (layer "F.Cu") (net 7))
 (via (at 134 82.75) (size 0.6) (drill 0.3) (layers "F.Cu" "B.Cu") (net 7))
 (segment (start 137.37 79.38) (end 139.38 79.38) (width 0.2) (layer "B.Cu") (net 7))
 (segment (start 134 82.75) (end 137.37 79.38) (width 0.2) (layer "B.Cu") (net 7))
 (segment (start 135.75 93.25) (end 150.91 93.25) (width 0.2) (layer "F.Cu") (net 6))
 (segment (start 118.875 88.5) (end 131 88.5) (width 0.2) (layer "F.Cu") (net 6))
 (segment (start 131 88.5) (end 135.75 93.25) (width 0.2) (layer "F.Cu") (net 6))
 (segment (start 150.91 93.25) (end 154.62 89.54) (width 0.2) (layer "F.Cu") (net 6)))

